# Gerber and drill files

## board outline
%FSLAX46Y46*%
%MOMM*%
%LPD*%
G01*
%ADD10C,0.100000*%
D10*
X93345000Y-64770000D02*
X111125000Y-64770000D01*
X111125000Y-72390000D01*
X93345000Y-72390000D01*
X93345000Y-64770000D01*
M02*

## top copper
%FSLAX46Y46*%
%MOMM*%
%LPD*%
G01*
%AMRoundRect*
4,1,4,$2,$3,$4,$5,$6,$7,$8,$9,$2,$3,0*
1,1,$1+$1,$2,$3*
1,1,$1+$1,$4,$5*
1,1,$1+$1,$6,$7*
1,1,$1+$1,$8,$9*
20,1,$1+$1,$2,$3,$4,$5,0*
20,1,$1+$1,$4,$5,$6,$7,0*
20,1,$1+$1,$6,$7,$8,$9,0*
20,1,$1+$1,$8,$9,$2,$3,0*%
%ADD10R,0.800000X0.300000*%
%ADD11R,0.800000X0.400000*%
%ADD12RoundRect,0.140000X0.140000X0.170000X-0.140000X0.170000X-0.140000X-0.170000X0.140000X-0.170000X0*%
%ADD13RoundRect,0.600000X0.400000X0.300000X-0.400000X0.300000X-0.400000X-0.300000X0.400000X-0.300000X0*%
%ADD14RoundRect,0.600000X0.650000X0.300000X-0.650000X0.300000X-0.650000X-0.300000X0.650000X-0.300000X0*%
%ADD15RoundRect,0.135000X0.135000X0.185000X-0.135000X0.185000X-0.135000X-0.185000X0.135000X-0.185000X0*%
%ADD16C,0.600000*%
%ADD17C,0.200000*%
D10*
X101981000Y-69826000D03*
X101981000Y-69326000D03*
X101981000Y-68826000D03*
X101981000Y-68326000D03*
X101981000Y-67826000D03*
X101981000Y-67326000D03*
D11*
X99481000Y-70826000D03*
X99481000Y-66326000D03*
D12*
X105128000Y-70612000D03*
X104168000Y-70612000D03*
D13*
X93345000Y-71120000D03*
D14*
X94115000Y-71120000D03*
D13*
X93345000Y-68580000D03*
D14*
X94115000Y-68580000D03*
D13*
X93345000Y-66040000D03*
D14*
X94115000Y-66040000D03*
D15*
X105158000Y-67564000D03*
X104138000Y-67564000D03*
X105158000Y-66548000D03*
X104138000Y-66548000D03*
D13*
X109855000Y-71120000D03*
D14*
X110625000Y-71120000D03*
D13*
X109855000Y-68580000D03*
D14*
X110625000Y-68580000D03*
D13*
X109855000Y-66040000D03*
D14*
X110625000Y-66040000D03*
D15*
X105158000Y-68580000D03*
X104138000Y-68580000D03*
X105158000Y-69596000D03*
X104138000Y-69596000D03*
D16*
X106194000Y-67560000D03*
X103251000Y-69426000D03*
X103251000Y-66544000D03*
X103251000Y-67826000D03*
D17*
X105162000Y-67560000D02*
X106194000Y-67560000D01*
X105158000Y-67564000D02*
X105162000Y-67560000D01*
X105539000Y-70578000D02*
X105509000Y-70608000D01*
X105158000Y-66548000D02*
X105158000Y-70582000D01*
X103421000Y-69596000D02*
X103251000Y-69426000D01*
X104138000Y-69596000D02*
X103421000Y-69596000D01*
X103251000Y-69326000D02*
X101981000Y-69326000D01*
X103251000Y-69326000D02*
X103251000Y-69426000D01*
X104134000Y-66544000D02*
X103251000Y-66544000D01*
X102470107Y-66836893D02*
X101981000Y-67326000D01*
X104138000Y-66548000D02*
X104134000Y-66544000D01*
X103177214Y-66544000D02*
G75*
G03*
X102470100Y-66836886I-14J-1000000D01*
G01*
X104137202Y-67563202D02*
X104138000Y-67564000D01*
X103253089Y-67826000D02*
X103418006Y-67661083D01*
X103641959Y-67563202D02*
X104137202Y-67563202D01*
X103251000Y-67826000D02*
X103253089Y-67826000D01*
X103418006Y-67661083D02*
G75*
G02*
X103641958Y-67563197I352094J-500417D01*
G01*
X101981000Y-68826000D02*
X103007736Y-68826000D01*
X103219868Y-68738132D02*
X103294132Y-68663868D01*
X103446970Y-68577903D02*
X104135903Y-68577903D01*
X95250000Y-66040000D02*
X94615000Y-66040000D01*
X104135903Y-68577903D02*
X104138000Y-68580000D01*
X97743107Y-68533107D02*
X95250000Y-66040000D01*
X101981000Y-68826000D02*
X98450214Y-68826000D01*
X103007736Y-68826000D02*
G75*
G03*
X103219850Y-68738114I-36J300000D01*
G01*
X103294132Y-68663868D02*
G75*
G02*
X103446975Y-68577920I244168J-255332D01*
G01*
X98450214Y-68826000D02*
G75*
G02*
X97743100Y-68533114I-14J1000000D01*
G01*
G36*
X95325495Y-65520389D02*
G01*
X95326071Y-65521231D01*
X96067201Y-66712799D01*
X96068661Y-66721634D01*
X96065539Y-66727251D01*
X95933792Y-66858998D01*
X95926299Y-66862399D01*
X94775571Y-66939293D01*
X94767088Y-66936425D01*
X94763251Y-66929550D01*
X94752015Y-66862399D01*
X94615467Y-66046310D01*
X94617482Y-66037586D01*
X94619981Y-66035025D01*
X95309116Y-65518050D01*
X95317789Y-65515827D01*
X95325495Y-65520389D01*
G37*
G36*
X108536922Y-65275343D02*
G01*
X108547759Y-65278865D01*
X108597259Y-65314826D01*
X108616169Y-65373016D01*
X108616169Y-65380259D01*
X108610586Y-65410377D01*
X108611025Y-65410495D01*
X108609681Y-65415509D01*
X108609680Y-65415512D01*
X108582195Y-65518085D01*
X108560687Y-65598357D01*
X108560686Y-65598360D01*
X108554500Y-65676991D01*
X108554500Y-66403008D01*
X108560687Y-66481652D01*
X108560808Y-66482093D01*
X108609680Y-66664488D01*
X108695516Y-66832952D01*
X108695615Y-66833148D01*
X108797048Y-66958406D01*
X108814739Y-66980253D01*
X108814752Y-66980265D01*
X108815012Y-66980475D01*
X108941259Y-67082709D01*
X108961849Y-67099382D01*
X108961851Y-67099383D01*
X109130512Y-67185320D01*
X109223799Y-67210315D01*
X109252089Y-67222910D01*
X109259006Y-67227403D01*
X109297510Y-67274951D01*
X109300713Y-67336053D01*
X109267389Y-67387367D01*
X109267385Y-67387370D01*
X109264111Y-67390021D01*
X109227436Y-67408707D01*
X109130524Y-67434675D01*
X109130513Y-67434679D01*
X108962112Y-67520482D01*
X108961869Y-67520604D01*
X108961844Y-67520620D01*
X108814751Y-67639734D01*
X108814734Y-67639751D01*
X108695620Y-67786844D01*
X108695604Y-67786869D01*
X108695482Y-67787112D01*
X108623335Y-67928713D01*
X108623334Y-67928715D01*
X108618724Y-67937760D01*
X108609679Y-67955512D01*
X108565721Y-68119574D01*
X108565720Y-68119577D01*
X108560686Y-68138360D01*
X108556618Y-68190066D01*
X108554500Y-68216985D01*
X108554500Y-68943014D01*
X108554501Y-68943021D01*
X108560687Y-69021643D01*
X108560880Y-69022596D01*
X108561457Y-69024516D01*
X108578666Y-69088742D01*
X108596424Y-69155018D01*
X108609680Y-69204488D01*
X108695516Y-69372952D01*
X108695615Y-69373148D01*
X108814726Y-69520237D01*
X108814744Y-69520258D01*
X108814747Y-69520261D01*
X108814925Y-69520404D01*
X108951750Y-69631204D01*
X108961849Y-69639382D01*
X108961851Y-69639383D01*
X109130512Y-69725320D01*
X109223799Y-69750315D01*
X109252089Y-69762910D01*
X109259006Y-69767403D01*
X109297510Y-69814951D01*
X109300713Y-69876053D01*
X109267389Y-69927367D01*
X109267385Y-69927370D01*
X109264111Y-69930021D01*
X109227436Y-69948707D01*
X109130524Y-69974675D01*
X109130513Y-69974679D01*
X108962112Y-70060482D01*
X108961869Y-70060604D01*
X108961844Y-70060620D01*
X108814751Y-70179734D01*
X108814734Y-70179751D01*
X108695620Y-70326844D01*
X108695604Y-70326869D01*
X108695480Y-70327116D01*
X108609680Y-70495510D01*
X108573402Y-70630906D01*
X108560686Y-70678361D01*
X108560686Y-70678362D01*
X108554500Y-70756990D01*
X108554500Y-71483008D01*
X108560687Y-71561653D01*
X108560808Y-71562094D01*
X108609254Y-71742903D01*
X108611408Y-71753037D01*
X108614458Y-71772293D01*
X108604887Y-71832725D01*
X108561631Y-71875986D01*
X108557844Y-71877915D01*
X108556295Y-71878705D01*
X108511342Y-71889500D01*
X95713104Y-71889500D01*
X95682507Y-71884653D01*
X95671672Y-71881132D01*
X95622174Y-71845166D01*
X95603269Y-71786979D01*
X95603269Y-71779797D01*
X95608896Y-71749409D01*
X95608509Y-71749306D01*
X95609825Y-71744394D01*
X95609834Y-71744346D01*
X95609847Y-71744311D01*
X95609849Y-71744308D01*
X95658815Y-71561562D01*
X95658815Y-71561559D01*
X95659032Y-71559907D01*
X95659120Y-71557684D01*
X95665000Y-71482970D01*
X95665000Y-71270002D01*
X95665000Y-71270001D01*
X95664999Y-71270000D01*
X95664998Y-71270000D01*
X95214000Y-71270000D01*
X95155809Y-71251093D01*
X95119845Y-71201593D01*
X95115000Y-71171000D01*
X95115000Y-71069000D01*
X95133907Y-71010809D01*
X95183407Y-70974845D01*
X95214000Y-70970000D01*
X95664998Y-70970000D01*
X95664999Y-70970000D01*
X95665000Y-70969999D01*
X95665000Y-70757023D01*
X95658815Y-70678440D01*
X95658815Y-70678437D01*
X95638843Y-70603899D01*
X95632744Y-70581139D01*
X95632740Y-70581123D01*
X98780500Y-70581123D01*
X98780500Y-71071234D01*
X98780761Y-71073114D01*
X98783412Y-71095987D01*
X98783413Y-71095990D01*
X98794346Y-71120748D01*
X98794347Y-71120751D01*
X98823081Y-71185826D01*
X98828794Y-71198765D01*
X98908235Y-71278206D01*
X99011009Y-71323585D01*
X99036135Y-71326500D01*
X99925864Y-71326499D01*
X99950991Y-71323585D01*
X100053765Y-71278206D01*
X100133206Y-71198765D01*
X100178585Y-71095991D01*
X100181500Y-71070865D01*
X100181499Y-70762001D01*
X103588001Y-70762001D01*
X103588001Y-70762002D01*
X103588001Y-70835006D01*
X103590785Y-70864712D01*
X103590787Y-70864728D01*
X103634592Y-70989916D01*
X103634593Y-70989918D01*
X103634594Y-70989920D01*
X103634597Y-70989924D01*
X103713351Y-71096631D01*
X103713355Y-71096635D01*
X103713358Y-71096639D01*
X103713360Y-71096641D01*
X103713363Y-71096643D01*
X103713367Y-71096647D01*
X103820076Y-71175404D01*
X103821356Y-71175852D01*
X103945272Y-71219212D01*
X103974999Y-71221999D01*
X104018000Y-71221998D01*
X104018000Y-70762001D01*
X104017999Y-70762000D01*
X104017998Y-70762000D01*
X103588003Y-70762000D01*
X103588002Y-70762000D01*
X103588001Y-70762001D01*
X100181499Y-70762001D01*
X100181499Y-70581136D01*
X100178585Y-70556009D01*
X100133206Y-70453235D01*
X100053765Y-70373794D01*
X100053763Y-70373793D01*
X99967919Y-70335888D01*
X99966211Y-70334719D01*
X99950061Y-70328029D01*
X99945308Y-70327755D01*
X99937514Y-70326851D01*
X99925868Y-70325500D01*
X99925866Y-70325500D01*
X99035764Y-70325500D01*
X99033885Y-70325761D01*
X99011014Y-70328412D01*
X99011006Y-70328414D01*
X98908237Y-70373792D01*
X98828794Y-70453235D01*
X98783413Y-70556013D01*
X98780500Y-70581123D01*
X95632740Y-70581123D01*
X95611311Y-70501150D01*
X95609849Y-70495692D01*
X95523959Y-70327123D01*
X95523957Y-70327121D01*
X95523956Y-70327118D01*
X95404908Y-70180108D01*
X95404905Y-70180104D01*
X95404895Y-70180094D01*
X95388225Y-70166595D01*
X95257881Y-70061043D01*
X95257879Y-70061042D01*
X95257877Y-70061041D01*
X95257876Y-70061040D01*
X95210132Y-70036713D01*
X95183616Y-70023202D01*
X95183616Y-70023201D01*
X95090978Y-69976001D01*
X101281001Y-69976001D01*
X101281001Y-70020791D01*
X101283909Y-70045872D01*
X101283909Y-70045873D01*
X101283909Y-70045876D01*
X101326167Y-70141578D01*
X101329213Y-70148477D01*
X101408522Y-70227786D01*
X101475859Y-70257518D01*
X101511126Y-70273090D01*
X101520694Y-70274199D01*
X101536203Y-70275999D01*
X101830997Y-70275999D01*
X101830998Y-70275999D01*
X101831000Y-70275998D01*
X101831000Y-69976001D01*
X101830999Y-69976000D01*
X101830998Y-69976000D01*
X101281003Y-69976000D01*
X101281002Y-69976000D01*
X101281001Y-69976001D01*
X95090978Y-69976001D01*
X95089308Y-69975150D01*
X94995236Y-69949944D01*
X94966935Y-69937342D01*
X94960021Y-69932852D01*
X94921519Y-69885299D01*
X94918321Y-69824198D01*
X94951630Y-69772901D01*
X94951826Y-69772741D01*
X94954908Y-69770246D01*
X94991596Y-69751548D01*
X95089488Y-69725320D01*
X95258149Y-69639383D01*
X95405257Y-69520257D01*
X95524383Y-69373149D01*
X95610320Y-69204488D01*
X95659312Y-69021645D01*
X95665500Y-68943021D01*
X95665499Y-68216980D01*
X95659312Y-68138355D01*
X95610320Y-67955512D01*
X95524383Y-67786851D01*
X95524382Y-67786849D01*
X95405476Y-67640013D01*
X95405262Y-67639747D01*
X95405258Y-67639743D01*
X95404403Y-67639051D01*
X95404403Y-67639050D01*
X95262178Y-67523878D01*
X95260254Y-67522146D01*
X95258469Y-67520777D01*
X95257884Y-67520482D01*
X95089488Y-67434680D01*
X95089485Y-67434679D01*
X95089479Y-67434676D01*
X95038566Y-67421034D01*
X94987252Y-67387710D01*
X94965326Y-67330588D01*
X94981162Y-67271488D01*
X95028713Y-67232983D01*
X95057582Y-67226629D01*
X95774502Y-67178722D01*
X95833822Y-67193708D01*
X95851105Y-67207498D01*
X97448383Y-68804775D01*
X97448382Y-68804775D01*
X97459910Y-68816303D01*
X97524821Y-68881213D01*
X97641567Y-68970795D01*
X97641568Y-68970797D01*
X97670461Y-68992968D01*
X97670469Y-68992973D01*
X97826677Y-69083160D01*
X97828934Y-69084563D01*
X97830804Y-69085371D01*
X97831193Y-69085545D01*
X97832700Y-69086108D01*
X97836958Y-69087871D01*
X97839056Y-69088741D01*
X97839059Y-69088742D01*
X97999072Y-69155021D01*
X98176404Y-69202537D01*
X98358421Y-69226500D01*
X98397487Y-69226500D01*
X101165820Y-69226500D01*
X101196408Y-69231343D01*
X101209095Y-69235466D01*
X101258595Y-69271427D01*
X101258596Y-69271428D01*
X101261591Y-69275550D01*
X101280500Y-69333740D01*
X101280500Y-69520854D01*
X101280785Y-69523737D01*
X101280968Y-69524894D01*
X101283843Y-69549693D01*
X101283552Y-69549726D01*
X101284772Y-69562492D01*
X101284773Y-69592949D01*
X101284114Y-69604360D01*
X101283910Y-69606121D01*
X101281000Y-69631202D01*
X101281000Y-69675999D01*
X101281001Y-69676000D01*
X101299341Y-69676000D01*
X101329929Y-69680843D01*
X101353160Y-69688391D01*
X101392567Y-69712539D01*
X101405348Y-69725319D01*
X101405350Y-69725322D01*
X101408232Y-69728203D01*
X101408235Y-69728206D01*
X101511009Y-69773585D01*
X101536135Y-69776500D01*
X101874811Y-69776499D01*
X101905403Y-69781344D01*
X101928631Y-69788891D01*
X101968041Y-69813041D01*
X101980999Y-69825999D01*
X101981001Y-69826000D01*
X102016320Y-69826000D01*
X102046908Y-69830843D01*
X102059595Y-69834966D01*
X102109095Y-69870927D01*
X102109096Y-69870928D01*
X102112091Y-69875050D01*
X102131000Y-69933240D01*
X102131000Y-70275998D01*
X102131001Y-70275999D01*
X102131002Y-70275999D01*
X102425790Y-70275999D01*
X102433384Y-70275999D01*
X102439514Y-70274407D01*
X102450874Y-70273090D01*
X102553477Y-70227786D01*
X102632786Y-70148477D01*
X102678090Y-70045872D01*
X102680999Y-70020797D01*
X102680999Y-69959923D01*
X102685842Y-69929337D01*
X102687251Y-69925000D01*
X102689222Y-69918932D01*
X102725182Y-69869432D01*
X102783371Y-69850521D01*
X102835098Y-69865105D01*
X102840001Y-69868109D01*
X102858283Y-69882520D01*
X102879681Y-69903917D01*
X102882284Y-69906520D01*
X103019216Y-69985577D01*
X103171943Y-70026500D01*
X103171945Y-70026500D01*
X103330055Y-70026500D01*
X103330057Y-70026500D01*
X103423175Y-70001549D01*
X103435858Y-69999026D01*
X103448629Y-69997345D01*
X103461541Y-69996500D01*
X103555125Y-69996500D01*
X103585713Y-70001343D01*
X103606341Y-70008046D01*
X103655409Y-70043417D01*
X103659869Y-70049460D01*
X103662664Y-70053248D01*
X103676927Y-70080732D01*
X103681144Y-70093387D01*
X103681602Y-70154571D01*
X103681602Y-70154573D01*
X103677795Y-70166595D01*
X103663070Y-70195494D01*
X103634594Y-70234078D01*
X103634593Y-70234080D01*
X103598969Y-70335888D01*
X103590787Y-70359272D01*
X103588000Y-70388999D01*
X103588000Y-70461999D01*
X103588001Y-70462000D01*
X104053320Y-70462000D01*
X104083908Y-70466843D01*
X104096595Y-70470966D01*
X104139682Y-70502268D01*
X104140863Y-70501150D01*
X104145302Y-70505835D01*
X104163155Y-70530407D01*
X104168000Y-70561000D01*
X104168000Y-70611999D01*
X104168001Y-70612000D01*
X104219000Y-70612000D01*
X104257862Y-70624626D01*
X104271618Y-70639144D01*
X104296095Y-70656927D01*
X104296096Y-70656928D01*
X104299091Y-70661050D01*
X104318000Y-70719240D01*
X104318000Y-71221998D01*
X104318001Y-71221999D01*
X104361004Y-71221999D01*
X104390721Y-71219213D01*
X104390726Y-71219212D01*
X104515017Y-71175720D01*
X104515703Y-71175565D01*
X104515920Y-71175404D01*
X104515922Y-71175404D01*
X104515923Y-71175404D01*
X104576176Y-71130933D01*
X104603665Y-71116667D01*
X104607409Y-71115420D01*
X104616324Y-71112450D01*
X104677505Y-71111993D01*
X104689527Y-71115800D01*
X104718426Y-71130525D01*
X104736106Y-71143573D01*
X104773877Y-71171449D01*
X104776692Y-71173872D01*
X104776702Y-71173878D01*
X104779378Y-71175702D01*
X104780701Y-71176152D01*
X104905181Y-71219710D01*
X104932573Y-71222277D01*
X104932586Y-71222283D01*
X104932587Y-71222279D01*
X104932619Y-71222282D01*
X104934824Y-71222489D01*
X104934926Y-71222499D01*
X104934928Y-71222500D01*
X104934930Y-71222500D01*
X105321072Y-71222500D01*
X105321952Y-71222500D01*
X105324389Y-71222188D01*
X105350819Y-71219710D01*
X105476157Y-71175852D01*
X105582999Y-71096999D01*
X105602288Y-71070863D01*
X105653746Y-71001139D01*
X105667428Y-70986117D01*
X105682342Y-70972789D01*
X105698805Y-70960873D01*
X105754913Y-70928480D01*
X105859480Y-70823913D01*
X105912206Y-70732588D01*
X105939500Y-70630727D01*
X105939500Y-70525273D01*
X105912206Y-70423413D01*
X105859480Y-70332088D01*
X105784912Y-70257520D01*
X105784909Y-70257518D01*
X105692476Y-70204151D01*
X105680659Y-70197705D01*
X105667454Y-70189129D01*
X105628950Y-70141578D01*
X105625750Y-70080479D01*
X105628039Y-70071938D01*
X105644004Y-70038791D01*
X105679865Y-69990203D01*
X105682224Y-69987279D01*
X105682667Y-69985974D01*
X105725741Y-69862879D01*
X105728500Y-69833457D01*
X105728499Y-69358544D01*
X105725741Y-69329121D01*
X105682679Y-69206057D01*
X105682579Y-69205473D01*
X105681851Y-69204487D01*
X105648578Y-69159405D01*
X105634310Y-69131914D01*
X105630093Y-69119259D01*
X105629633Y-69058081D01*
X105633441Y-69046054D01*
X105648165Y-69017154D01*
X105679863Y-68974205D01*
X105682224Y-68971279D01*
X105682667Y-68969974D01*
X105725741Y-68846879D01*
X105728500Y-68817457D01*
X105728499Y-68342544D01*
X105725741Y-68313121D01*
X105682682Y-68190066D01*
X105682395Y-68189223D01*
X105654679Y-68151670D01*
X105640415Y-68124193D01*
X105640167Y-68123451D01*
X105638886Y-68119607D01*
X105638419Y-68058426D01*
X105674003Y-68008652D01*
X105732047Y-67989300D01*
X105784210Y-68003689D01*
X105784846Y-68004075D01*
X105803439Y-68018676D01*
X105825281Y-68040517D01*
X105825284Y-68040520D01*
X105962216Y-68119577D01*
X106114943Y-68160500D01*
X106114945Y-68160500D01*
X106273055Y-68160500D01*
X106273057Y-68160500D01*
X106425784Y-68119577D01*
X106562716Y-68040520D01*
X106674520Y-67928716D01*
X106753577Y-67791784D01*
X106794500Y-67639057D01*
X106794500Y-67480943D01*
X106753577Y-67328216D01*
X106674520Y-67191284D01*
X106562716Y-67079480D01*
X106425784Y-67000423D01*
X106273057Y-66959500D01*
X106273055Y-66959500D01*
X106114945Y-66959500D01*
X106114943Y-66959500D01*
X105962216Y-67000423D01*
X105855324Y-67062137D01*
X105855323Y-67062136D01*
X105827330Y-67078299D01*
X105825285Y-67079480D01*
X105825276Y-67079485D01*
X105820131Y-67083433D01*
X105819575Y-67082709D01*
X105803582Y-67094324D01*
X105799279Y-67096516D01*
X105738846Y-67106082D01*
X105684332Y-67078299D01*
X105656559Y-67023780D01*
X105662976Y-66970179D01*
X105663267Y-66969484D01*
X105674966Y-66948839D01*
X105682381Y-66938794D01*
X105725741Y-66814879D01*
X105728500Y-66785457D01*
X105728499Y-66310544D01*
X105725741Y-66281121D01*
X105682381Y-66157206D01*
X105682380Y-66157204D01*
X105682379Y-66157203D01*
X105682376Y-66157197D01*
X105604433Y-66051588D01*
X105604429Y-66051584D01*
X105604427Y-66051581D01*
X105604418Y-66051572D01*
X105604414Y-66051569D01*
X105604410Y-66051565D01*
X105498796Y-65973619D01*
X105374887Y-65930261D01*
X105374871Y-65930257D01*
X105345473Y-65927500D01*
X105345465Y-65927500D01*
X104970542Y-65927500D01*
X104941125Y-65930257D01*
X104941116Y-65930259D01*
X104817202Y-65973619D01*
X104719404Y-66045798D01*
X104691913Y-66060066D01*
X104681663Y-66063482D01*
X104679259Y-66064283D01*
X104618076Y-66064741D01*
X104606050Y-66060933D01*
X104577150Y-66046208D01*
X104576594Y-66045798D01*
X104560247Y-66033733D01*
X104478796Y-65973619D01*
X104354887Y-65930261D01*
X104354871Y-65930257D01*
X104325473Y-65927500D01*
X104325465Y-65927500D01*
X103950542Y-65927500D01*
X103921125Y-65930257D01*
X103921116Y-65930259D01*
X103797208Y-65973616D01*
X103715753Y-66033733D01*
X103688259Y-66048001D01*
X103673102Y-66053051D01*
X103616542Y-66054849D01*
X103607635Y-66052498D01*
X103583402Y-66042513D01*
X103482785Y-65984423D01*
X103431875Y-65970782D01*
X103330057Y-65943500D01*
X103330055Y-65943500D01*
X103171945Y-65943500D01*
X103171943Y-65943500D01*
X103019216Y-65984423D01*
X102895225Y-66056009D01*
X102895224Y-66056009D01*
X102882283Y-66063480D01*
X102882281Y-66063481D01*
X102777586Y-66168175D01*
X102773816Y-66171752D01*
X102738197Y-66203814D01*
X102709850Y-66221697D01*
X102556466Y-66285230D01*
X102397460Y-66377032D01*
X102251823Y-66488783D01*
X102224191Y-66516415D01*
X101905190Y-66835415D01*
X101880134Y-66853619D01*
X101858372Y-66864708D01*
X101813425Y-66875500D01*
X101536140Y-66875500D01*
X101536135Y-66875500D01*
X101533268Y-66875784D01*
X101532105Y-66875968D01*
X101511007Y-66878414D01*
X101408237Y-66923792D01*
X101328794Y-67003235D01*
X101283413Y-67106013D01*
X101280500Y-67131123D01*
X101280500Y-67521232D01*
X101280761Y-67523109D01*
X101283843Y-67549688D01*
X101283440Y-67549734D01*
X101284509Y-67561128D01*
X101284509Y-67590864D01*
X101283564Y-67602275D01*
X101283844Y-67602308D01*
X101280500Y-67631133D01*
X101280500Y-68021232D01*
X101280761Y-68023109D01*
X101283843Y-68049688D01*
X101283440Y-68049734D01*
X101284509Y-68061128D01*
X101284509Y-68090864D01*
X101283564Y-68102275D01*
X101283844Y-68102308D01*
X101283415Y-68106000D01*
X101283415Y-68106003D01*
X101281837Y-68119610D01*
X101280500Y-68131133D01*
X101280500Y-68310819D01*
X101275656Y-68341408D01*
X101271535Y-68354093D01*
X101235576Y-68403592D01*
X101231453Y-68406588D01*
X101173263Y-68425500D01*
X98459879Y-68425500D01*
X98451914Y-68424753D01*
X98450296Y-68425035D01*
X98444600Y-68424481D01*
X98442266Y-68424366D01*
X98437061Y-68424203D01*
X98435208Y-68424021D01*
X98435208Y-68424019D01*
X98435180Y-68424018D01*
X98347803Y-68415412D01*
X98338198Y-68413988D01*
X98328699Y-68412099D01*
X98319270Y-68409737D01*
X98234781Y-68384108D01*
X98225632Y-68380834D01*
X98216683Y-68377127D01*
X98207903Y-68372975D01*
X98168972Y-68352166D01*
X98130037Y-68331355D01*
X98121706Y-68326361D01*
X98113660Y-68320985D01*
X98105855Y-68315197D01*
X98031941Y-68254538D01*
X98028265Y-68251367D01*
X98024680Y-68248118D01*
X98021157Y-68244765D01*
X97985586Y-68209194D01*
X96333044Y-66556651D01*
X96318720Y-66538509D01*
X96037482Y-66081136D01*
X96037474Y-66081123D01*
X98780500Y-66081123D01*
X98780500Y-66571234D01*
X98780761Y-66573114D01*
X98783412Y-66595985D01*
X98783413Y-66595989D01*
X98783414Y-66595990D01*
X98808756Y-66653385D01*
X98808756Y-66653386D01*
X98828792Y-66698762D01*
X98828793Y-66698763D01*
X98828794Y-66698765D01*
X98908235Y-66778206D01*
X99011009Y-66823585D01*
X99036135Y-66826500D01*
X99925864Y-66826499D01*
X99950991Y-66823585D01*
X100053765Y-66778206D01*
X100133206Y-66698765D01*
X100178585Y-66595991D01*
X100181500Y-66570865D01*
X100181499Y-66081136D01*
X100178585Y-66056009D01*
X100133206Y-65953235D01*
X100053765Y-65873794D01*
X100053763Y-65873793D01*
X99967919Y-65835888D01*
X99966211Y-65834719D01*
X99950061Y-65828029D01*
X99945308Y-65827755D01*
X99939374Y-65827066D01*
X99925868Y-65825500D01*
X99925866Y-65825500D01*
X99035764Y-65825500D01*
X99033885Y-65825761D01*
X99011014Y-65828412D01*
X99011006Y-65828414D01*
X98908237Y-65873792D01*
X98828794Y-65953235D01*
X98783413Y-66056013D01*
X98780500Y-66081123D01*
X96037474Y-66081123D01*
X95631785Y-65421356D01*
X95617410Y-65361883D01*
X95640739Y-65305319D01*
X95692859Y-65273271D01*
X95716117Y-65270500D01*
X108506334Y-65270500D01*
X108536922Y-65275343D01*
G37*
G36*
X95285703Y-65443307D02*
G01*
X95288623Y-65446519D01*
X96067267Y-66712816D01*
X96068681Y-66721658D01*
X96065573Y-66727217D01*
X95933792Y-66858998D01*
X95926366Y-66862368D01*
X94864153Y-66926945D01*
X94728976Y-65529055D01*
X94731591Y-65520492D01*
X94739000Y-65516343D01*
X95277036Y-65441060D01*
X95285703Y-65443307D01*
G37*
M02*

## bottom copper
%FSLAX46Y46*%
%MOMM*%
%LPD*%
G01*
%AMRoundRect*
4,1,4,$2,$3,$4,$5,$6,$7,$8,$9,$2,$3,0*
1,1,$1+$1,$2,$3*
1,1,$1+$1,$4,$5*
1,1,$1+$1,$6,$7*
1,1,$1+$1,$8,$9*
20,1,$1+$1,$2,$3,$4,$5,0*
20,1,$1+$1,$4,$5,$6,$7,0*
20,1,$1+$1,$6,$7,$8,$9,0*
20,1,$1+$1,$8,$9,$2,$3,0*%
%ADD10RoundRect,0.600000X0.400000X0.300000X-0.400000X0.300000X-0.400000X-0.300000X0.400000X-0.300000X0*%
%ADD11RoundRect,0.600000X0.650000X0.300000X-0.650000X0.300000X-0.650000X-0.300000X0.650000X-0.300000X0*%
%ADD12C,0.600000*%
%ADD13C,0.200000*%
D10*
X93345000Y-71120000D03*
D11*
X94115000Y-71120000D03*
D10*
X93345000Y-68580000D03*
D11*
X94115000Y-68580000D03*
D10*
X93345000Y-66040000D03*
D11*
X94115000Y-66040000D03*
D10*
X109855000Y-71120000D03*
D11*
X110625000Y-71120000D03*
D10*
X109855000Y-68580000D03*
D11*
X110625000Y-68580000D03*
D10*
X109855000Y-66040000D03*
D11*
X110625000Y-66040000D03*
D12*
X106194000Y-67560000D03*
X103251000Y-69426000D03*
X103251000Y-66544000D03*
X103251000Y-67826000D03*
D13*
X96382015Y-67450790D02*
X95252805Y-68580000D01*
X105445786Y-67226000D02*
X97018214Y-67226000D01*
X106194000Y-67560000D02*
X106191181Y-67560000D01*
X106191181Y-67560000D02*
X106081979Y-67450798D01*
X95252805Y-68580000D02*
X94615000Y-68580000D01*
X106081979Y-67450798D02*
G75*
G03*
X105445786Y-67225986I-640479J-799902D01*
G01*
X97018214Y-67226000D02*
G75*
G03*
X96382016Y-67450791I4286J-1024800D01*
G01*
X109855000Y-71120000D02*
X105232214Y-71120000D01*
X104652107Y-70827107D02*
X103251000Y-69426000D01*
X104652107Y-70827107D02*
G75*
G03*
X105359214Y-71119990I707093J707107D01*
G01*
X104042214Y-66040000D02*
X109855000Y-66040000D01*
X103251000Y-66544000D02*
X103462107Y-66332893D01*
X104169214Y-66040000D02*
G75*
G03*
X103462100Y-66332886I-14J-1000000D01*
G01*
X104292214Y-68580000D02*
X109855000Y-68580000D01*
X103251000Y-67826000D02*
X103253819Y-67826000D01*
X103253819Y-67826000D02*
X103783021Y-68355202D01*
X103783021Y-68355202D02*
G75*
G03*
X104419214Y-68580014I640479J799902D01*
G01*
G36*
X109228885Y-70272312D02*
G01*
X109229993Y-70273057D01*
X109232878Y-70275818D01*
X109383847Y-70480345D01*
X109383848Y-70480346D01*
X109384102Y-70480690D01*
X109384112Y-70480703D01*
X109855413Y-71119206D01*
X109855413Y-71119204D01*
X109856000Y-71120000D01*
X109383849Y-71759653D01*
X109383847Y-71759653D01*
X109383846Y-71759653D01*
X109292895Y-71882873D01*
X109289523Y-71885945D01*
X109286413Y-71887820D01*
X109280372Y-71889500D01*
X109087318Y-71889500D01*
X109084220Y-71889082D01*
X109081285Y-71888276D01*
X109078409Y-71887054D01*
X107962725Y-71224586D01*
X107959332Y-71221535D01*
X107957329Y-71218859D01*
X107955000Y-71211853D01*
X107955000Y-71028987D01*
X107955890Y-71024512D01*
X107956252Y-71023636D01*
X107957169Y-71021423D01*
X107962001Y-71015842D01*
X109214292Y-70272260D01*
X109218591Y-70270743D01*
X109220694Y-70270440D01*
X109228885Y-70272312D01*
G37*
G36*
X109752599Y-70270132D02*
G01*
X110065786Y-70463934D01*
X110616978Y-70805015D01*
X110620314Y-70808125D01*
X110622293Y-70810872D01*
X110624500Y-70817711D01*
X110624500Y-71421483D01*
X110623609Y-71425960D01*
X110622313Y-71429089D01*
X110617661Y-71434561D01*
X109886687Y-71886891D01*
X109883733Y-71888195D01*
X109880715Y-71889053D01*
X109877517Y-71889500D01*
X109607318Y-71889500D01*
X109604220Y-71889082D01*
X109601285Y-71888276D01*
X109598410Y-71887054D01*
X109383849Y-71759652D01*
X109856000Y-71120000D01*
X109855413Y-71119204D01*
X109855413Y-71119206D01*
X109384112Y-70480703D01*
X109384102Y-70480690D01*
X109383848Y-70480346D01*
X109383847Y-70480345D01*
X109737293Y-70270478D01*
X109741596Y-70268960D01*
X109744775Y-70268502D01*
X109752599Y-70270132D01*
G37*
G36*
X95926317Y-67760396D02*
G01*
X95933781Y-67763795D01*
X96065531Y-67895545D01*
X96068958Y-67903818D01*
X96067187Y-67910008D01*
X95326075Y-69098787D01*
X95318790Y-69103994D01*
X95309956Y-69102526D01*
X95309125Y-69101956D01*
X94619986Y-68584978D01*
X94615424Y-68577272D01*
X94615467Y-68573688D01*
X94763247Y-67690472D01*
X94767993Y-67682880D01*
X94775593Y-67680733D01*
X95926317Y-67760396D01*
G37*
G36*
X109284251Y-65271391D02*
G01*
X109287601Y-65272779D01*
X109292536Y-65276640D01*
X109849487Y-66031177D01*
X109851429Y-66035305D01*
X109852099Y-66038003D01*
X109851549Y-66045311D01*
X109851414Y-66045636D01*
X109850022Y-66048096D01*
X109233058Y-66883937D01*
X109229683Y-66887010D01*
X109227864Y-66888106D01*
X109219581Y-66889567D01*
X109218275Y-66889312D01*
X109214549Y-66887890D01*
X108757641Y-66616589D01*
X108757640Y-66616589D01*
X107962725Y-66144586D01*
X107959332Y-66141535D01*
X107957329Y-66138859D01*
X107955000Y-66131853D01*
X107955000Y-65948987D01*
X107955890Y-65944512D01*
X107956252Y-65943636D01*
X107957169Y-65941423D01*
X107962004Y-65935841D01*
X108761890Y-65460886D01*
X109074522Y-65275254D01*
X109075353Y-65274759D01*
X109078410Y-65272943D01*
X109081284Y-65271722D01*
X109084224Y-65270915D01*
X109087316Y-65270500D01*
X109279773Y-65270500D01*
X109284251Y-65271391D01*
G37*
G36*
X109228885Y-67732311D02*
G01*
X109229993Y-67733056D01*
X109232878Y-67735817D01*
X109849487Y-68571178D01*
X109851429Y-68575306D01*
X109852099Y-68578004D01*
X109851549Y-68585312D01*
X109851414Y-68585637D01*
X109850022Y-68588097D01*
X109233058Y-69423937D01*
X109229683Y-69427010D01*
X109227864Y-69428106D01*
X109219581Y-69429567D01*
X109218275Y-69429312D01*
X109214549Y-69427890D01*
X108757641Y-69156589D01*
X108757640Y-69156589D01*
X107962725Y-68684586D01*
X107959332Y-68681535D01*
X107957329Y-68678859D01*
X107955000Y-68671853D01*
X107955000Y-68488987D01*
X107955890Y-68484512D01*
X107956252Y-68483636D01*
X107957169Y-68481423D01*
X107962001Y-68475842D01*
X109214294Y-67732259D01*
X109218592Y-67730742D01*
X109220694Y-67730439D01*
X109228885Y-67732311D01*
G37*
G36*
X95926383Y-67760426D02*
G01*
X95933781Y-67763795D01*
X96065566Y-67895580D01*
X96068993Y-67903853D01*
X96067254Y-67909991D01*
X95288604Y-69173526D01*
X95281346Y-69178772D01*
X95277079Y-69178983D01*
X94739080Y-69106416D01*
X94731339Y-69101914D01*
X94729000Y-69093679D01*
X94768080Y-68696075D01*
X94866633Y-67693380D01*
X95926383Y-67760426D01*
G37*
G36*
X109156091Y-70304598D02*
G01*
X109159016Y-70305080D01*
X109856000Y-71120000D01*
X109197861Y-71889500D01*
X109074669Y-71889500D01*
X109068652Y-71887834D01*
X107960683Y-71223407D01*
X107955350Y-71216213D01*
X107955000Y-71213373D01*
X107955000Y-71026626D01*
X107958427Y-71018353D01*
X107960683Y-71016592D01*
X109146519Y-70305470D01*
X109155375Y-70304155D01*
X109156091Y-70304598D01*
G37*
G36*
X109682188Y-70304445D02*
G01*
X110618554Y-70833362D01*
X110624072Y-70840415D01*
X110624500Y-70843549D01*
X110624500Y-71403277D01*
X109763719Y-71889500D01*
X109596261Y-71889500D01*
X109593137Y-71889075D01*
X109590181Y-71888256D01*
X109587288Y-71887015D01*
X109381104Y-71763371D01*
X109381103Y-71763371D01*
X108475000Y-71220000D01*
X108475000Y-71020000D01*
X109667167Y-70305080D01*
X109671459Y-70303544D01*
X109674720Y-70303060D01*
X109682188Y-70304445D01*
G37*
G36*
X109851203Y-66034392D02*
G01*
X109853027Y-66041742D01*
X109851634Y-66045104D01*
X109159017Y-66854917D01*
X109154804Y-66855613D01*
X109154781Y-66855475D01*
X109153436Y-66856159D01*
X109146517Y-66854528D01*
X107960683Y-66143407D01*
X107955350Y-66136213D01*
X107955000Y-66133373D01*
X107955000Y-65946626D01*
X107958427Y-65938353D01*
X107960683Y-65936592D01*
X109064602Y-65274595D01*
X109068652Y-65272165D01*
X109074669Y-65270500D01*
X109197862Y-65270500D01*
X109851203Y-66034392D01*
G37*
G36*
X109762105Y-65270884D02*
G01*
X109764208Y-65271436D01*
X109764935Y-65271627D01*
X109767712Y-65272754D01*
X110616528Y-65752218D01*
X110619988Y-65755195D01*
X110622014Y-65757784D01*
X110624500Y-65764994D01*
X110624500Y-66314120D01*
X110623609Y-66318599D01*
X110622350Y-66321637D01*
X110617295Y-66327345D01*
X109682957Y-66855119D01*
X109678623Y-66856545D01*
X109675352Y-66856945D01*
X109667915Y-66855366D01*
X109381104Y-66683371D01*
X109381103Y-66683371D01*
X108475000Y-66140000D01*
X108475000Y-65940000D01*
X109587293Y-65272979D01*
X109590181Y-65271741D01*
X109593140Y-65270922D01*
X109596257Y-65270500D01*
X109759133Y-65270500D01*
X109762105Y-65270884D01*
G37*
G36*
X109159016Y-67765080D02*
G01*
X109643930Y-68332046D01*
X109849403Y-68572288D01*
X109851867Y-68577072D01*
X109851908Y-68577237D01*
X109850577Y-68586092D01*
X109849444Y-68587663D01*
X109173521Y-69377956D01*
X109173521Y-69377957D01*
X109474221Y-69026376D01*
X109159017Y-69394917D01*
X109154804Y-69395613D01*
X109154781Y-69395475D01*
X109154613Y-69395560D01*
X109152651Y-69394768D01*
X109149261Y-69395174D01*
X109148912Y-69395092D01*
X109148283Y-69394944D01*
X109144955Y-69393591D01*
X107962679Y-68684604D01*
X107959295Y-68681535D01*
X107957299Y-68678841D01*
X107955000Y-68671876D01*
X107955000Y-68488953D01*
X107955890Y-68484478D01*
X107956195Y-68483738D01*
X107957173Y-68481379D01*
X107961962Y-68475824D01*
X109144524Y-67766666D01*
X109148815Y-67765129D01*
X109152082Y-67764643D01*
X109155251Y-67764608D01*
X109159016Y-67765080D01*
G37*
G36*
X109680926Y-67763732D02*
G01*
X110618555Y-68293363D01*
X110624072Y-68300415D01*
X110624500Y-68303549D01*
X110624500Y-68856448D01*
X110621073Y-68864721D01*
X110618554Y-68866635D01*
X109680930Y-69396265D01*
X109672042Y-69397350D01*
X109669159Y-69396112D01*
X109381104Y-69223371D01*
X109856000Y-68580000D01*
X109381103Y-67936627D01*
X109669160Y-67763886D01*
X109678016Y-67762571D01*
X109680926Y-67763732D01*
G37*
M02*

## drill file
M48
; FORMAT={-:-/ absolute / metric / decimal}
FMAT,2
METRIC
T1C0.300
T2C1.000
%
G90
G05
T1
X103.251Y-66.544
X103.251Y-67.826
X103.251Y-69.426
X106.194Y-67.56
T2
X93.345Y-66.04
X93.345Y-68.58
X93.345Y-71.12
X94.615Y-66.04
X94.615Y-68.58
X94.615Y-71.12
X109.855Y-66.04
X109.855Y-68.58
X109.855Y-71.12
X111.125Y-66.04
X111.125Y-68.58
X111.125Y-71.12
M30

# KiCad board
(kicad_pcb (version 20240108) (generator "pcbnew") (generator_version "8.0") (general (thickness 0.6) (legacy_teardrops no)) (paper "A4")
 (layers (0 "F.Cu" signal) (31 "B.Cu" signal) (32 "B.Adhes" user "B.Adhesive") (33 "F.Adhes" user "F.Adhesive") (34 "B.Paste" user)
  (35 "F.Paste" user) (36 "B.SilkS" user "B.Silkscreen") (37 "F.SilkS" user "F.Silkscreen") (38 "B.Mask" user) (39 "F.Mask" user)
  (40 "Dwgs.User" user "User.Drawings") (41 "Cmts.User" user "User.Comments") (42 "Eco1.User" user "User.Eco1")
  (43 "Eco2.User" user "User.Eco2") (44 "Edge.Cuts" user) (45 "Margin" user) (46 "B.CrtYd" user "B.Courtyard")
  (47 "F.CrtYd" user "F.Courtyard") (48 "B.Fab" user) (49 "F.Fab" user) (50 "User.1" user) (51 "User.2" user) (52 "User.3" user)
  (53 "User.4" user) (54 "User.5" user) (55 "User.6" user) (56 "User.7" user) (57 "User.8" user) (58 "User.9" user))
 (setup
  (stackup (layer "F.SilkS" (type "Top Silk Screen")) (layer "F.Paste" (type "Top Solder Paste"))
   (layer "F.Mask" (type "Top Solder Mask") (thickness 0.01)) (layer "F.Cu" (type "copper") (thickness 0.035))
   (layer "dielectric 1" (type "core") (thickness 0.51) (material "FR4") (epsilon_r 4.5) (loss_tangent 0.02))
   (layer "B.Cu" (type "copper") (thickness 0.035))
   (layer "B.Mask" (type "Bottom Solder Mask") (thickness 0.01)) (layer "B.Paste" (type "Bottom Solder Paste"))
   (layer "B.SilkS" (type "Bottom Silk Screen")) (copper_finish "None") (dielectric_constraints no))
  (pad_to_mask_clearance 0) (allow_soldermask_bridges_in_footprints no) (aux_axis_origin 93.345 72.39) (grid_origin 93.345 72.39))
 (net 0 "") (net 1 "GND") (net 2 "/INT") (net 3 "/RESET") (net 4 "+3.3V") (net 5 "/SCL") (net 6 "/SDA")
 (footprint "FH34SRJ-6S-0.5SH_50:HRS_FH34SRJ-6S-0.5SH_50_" (layer "F.Cu") (at 100.731 68.576 -90)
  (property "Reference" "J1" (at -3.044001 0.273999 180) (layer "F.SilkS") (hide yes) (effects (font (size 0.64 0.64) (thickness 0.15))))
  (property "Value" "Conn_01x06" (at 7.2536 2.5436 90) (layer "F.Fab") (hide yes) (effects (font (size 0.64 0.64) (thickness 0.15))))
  (pad "1" smd rect (at 1.25 -1.25 270) (size 0.3 0.8) (layers "F.Cu" "F.Mask") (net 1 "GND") (solder_mask_margin 0.102)
   (teardrops (best_length_ratio 1) (max_length 1) (best_width_ratio 1) (max_width 2) (curve_points 10) (filter_ratio 0.9) (enabled no)
    (allow_two_segments yes) (prefer_zone_connections yes)))
  (pad "2" smd rect (at 0.75 -1.25 270) (size 0.3 0.8) (layers "F.Cu" "F.Mask") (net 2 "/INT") (solder_mask_margin 0.102)
   (teardrops (best_length_ratio 1) (max_length 1) (best_width_ratio 1) (max_width 2) (curve_points 10) (filter_ratio 0.9) (enabled no)
    (allow_two_segments yes) (prefer_zone_connections yes)))
  (pad "3" smd rect (at 0.25 -1.25 270) (size 0.3 0.8) (layers "F.Cu" "F.Mask") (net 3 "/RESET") (solder_mask_margin 0.102)
   (teardrops (best_length_ratio 1) (max_length 1) (best_width_ratio 1) (max_width 2) (curve_points 10) (filter_ratio 0.9) (enabled no)
    (allow_two_segments yes) (prefer_zone_connections yes)))
  (pad "4" smd rect (at -0.25 -1.25 270) (size 0.3 0.8) (layers "F.Cu" "F.Mask") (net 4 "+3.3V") (solder_mask_margin 0.102)
   (teardrops (best_length_ratio 1) (max_length 1) (best_width_ratio 1) (max_width 2) (curve_points 10) (filter_ratio 0.9) (enabled no)
    (allow_two_segments yes) (prefer_zone_connections yes)))
  (pad "5" smd rect (at -0.75 -1.25 270) (size 0.3 0.8) (layers "F.Cu" "F.Mask") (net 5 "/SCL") (solder_mask_margin 0.102)
   (teardrops (best_length_ratio 1) (max_length 1) (best_width_ratio 1) (max_width 2) (curve_points 10) (filter_ratio 0.9) (enabled no)
    (allow_two_segments yes) (prefer_zone_connections yes)))
  (pad "6" smd rect (at -1.25 -1.25 270) (size 0.3 0.8) (layers "F.Cu" "F.Mask") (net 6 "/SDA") (solder_mask_margin 0.102)
   (teardrops (best_length_ratio 1) (max_length 1) (best_width_ratio 1) (max_width 2) (curve_points 10) (filter_ratio 0.9) (enabled no)
    (allow_two_segments yes) (prefer_zone_connections yes)))
  (pad "S1" smd rect (at 2.25 1.25 270) (size 0.4 0.8) (layers "F.Cu" "F.Paste" "F.Mask") (solder_mask_margin 0.102)
   (teardrops (best_length_ratio 1) (max_length 1) (best_width_ratio 1) (max_width 2) (curve_points 10) (filter_ratio 0.9) (enabled no)
    (allow_two_segments yes) (prefer_zone_connections yes)))
  (pad "S2" smd rect (at -2.25 1.25 270) (size 0.4 0.8) (layers "F.Cu" "F.Paste" "F.Mask") (solder_mask_margin 0.102)
   (teardrops (best_length_ratio 1) (max_length 1) (best_width_ratio 1) (max_width 2) (curve_points 10) (filter_ratio 0.9) (enabled no)
    (allow_two_segments yes) (prefer_zone_connections yes))))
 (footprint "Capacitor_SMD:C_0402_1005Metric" (layer "F.Cu") (at 104.648 70.612 180)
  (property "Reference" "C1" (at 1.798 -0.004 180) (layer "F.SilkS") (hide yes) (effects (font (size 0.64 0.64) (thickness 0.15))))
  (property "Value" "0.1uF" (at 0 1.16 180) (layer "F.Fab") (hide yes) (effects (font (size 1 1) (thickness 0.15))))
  (pad "1" smd roundrect (at -0.48 0 180) (size 0.56 0.62) (layers "F.Cu" "F.Paste" "F.Mask") (roundrect_rratio 0.25) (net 4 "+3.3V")
   (teardrops (best_length_ratio 1) (max_length 1) (best_width_ratio 1) (max_width 2) (curve_points 10) (filter_ratio 0.9) (enabled no)
    (allow_two_segments yes) (prefer_zone_connections yes)))
  (pad "2" smd roundrect (at 0.48 0 180) (size 0.56 0.62) (layers "F.Cu" "F.Paste" "F.Mask") (roundrect_rratio 0.25) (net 1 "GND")
   (teardrops (best_length_ratio 1) (max_length 1) (best_width_ratio 1) (max_width 2) (curve_points 10) (filter_ratio 0.9) (enabled no)
    (allow_two_segments yes) (prefer_zone_connections yes))))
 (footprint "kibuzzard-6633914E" (layer "F.Cu") (at 107.442 71.12)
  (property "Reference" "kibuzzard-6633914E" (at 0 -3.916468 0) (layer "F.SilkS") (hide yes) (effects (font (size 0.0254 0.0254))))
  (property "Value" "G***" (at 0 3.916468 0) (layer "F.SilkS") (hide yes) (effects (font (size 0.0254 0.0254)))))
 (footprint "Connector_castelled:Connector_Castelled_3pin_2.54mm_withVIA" (layer "F.Cu") (at 93.345 71.12 90)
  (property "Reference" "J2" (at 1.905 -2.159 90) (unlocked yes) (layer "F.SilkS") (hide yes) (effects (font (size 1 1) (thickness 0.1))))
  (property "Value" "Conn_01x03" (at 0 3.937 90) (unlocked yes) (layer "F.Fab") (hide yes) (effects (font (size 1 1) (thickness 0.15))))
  (pad "1" thru_hole roundrect (at 0 0 180) (size 2 1.8) (drill 1) (layers "*.Cu" "*.Mask") (remove_unused_layers no)
   (roundrect_rratio 0.3333333333) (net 1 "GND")
   (teardrops (best_length_ratio 0.5) (max_length 1) (best_width_ratio 1) (max_width 2) (curve_points 0) (filter_ratio 0.9) (enabled yes)
    (allow_two_segments yes) (prefer_zone_connections yes)))
  (pad "1" thru_hole roundrect (at 0 1.27 180) (size 2.5 1.8) (drill 1 (offset 0.5 0)) (layers "*.Cu" "*.Mask") (remove_unused_layers no)
   (roundrect_rratio 0.3333333333) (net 1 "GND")
   (teardrops (best_length_ratio 0.5) (max_length 1) (best_width_ratio 1) (max_width 2) (curve_points 0) (filter_ratio 0.9) (enabled yes)
    (allow_two_segments yes) (prefer_zone_connections yes)))
  (pad "2" thru_hole roundrect (at 2.54 0 180) (size 2 1.8) (drill 1) (layers "*.Cu" "*.Mask") (remove_unused_layers no)
   (roundrect_rratio 0.3333333333) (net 4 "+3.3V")
   (teardrops (best_length_ratio 0.5) (max_length 1) (best_width_ratio 1) (max_width 2) (curve_points 0) (filter_ratio 0.9) (enabled yes)
    (allow_two_segments yes) (prefer_zone_connections yes)))
  (pad "2" thru_hole roundrect (at 2.54 1.27 180) (size 2.5 1.8) (drill 1 (offset 0.5 0)) (layers "*.Cu" "*.Mask") (remove_unused_layers no)
   (roundrect_rratio 0.3333333333) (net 4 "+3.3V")
   (teardrops (best_length_ratio 0.5) (max_length 1) (best_width_ratio 1) (max_width 2) (curve_points 0) (filter_ratio 0.9) (enabled yes)
    (allow_two_segments yes) (prefer_zone_connections yes)))
  (pad "3" thru_hole roundrect (at 5.08 0 180) (size 2 1.8) (drill 1) (layers "*.Cu" "*.Mask") (remove_unused_layers no)
   (roundrect_rratio 0.3333333333) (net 3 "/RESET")
   (teardrops (best_length_ratio 0.5) (max_length 1) (best_width_ratio 1) (max_width 2) (curve_points 0) (filter_ratio 0.9) (enabled yes)
    (allow_two_segments yes) (prefer_zone_connections yes)))
  (pad "3" thru_hole roundrect (at 5.08 1.27 180) (size 2.5 1.8) (drill 1 (offset 0.5 0)) (layers "*.Cu" "*.Mask") (remove_unused_layers no)
   (roundrect_rratio 0.3333333333) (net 3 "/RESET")
   (teardrops (best_length_ratio 0.5) (max_length 1) (best_width_ratio 1) (max_width 2) (curve_points 0) (filter_ratio 0.9) (enabled yes)
    (allow_two_segments yes) (prefer_zone_connections yes))))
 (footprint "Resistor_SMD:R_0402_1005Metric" (layer "F.Cu") (at 104.648 67.564 180)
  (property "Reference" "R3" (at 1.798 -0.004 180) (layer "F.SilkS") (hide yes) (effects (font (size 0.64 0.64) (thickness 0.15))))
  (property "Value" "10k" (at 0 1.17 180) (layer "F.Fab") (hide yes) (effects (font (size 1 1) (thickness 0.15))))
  (pad "1" smd roundrect (at -0.51 0 180) (size 0.54 0.64) (layers "F.Cu" "F.Paste" "F.Mask") (roundrect_rratio 0.25) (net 4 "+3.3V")
   (teardrops (best_length_ratio 1) (max_length 1) (best_width_ratio 1) (max_width 2) (curve_points 10) (filter_ratio 0.9) (enabled no)
    (allow_two_segments yes) (prefer_zone_connections yes)))
  (pad "2" smd roundrect (at 0.51 0 180) (size 0.54 0.64) (layers "F.Cu" "F.Paste" "F.Mask") (roundrect_rratio 0.25) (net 5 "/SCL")
   (teardrops (best_length_ratio 1) (max_length 1) (best_width_ratio 1) (max_width 2) (curve_points 10) (filter_ratio 0.9) (enabled no)
    (allow_two_segments yes) (prefer_zone_connections yes))))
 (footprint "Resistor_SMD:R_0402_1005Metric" (layer "F.Cu") (at 104.648 66.548 180)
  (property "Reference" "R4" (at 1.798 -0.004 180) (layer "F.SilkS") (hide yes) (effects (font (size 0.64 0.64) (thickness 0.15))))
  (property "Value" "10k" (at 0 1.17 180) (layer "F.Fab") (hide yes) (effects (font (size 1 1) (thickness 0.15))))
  (pad "1" smd roundrect (at -0.51 0 180) (size 0.54 0.64) (layers "F.Cu" "F.Paste" "F.Mask") (roundrect_rratio 0.25) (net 4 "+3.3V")
   (teardrops (best_length_ratio 1) (max_length 1) (best_width_ratio 1) (max_width 2) (curve_points 10) (filter_ratio 0.9) (enabled no)
    (allow_two_segments yes) (prefer_zone_connections yes)))
  (pad "2" smd roundrect (at 0.51 0 180) (size 0.54 0.64) (layers "F.Cu" "F.Paste" "F.Mask") (roundrect_rratio 0.25) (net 6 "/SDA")
   (teardrops (best_length_ratio 1) (max_length 1) (best_width_ratio 1) (max_width 2) (curve_points 10) (filter_ratio 0.9) (enabled no)
    (allow_two_segments yes) (prefer_zone_connections yes))))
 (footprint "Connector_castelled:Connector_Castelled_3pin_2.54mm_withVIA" (layer "F.Cu") (at 109.855 71.12 90)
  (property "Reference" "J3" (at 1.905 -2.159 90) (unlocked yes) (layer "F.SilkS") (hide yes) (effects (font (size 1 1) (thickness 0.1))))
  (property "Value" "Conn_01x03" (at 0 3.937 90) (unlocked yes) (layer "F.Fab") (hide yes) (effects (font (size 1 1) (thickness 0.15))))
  (pad "1" thru_hole roundrect (at 0 0 180) (size 2 1.8) (drill 1) (layers "*.Cu" "*.Mask") (remove_unused_layers no)
   (roundrect_rratio 0.3333333333) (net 2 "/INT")
   (teardrops (best_length_ratio 0.5) (max_length 1) (best_width_ratio 1) (max_width 2) (curve_points 0) (filter_ratio 0.9) (enabled yes)
    (allow_two_segments yes) (prefer_zone_connections yes)))
  (pad "1" thru_hole roundrect (at 0 1.27 180) (size 2.5 1.8) (drill 1 (offset 0.5 0)) (layers "*.Cu" "*.Mask") (remove_unused_layers no)
   (roundrect_rratio 0.3333333333) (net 2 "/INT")
   (teardrops (best_length_ratio 0.5) (max_length 1) (best_width_ratio 1) (max_width 2) (curve_points 0) (filter_ratio 0.9) (enabled yes)
    (allow_two_segments yes) (prefer_zone_connections yes)))
  (pad "2" thru_hole roundrect (at 2.54 0 180) (size 2 1.8) (drill 1) (layers "*.Cu" "*.Mask") (remove_unused_layers no)
   (roundrect_rratio 0.3333333333) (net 5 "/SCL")
   (teardrops (best_length_ratio 0.5) (max_length 1) (best_width_ratio 1) (max_width 2) (curve_points 0) (filter_ratio 0.9) (enabled yes)
    (allow_two_segments yes) (prefer_zone_connections yes)))
  (pad "2" thru_hole roundrect (at 2.54 1.27 180) (size 2.5 1.8) (drill 1 (offset 0.5 0)) (layers "*.Cu" "*.Mask") (remove_unused_layers no)
   (roundrect_rratio 0.3333333333) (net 5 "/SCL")
   (teardrops (best_length_ratio 0.5) (max_length 1) (best_width_ratio 1) (max_width 2) (curve_points 0) (filter_ratio 0.9) (enabled yes)
    (allow_two_segments yes) (prefer_zone_connections yes)))
  (pad "3" thru_hole roundrect (at 5.08 0 180) (size 2 1.8) (drill 1) (layers "*.Cu" "*.Mask") (remove_unused_layers no)
   (roundrect_rratio 0.3333333333) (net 6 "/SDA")
   (teardrops (best_length_ratio 0.5) (max_length 1) (best_width_ratio 1) (max_width 2) (curve_points 0) (filter_ratio 0.9) (enabled yes)
    (allow_two_segments yes) (prefer_zone_connections yes)))
  (pad "3" thru_hole roundrect (at 5.08 1.27 180) (size 2.5 1.8) (drill 1 (offset 0.5 0)) (layers "*.Cu" "*.Mask") (remove_unused_layers no)
   (roundrect_rratio 0.3333333333) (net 6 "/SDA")
   (teardrops (best_length_ratio 0.5) (max_length 1) (best_width_ratio 1) (max_width 2) (curve_points 0) (filter_ratio 0.9) (enabled yes)
    (allow_two_segments yes) (prefer_zone_connections yes))))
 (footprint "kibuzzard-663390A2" (layer "F.Cu") (at 96.774 66.04)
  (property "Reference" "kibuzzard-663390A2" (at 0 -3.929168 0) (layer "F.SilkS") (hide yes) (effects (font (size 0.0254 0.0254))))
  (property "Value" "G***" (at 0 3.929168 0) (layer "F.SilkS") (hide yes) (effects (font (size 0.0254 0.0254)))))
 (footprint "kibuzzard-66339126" (layer "F.Cu") (at 107.442 68.58)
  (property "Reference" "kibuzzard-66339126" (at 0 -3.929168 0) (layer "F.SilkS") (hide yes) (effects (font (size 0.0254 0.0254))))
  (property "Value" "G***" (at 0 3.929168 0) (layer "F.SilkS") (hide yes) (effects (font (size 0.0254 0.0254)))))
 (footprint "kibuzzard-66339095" (layer "F.Cu") (at 96.901 71.12)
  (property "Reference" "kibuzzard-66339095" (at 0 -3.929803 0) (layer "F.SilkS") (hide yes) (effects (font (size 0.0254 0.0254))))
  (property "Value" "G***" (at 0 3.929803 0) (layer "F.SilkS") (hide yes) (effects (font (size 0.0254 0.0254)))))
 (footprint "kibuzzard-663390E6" (layer "F.Cu") (at 107.442 66.04)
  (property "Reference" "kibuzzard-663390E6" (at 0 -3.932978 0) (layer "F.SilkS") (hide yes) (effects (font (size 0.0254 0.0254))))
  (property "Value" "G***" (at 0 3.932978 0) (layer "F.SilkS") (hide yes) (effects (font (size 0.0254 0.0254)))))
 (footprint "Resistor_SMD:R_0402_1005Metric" (layer "F.Cu") (at 104.648 68.58 180)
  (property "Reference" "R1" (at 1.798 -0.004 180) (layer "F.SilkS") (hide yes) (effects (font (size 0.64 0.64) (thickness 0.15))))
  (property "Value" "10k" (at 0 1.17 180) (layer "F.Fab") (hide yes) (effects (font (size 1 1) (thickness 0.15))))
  (pad "1" smd roundrect (at -0.51 0 180) (size 0.54 0.64) (layers "F.Cu" "F.Paste" "F.Mask") (roundrect_rratio 0.25) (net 4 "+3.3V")
   (teardrops (best_length_ratio 1) (max_length 1) (best_width_ratio 1) (max_width 2) (curve_points 10) (filter_ratio 0.9) (enabled no)
    (allow_two_segments yes) (prefer_zone_connections yes)))
  (pad "2" smd roundrect (at 0.51 0 180) (size 0.54 0.64) (layers "F.Cu" "F.Paste" "F.Mask") (roundrect_rratio 0.25) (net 3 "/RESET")
   (teardrops (best_length_ratio 1) (max_length 1) (best_width_ratio 1) (max_width 2) (curve_points 10) (filter_ratio 0.9) (enabled no)
    (allow_two_segments yes) (prefer_zone_connections yes))))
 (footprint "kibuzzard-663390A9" (layer "F.Cu") (at 96.774 68.58)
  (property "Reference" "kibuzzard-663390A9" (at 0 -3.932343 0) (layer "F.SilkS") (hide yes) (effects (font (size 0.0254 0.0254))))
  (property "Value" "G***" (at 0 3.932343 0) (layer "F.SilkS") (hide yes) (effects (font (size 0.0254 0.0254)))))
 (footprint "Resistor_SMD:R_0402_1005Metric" (layer "F.Cu") (at 104.648 69.596 180)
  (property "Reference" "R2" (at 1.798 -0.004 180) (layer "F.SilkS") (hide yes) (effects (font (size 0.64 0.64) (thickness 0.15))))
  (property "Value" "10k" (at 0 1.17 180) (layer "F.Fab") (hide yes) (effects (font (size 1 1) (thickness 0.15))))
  (pad "1" smd roundrect (at -0.51 0 180) (size 0.54 0.64) (layers "F.Cu" "F.Paste" "F.Mask") (roundrect_rratio 0.25) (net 4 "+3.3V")
   (teardrops (best_length_ratio 1) (max_length 1) (best_width_ratio 1) (max_width 2) (curve_points 10) (filter_ratio 0.9) (enabled no)
    (allow_two_segments yes) (prefer_zone_connections yes)))
  (pad "2" smd roundrect (at 0.51 0 180) (size 0.54 0.64) (layers "F.Cu" "F.Paste" "F.Mask") (roundrect_rratio 0.25) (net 2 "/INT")
   (teardrops (best_length_ratio 1) (max_length 1) (best_width_ratio 1) (max_width 2) (curve_points 10) (filter_ratio 0.9) (enabled no)
    (allow_two_segments yes) (prefer_zone_connections yes))))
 (gr_rect (start 93.345 64.77) (end 111.125 72.39) (stroke (width 0.1) (type default)) (fill none) (layer "Edge.Cuts"))
 (segment (start 105.162 67.56) (end 106.194 67.56) (width 0.2) (layer "F.Cu") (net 4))
 (segment (start 105.158 67.564) (end 105.162 67.56) (width 0.2) (layer "F.Cu") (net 4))
 (segment (start 105.539 70.578) (end 105.509 70.608) (width 0.2) (layer "F.Cu") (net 4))
 (segment (start 105.158 66.548) (end 105.158 70.582) (width 0.2) (layer "F.Cu") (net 4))
 (via (at 106.194 67.56) (size 0.6) (drill 0.3) (layers "F.Cu" "B.Cu")
  (teardrops (best_length_ratio 1) (max_length 1) (best_width_ratio 1) (max_width 2) (curve_points 10) (filter_ratio 0.9) (enabled no)
   (allow_two_segments yes) (prefer_zone_connections yes))
  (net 4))
 (segment (start 96.382015 67.45079) (end 95.252805 68.58) (width 0.2) (layer "B.Cu") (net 4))
 (segment (start 105.445786 67.226) (end 97.018214 67.226) (width 0.2) (layer "B.Cu") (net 4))
 (segment (start 106.194 67.56) (end 106.191181 67.56) (width 0.2) (layer "B.Cu") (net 4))
 (segment (start 106.191181 67.56) (end 106.081979 67.450798) (width 0.2) (layer "B.Cu") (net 4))
 (segment (start 95.252805 68.58) (end 94.615 68.58) (width 0.2) (layer "B.Cu") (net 4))
 (arc (start 106.081979 67.450798) (mid 105.782679 67.284452) (end 105.445786 67.226) (width 0.2) (layer "B.Cu") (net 4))
 (arc (start 97.018214 67.226) (mid 96.681322 67.284452) (end 96.382015 67.45079) (width 0.2) (layer "B.Cu") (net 4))
 (segment (start 103.421 69.596) (end 103.251 69.426) (width 0.2) (layer "F.Cu") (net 2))
 (segment (start 104.138 69.596) (end 103.421 69.596) (width 0.2) (layer "F.Cu") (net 2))
 (segment (start 103.251 69.326) (end 101.981 69.326) (width 0.2) (layer "F.Cu") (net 2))
 (segment (start 103.251 69.326) (end 103.251 69.426) (width 0.2) (layer "F.Cu") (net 2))
 (via (at 103.251 69.426) (size 0.6) (drill 0.3) (layers "F.Cu" "B.Cu")
  (teardrops (best_length_ratio 1) (max_length 1) (best_width_ratio 1) (max_width 2) (curve_points 10) (filter_ratio 0.9) (enabled no)
   (allow_two_segments yes) (prefer_zone_connections yes))
  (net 2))
 (segment (start 109.855 71.12) (end 105.232214 71.12) (width 0.2) (layer "B.Cu") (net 2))
 (segment (start 104.652107 70.827107) (end 103.251 69.426) (width 0.2) (layer "B.Cu") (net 2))
 (arc (start 104.652107 70.827107) (mid 104.97653 71.04388) (end 105.359214 71.12) (width 0.2) (layer "B.Cu") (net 2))
 (segment (start 104.134 66.544) (end 103.251 66.544) (width 0.2) (layer "F.Cu") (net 6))
 (segment (start 102.470107 66.836893) (end 101.981 67.326) (width 0.2) (layer "F.Cu") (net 6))
 (segment (start 104.138 66.548) (end 104.134 66.544) (width 0.2) (layer "F.Cu") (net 6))
 (via (at 103.251 66.544) (size 0.6) (drill 0.3) (layers "F.Cu" "B.Cu")
  (teardrops (best_length_ratio 1) (max_length 1) (best_width_ratio 1) (max_width 2) (curve_points 10) (filter_ratio 0.9) (enabled no)
   (allow_two_segments yes) (prefer_zone_connections yes))
  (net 6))
 (arc (start 103.177214 66.544) (mid 102.794531 66.62012) (end 102.470107 66.836893) (width 0.2) (layer "F.Cu") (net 6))
 (segment (start 104.042214 66.04) (end 109.855 66.04) (width 0.2) (layer "B.Cu") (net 6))
 (segment (start 103.251 66.544) (end 103.462107 66.332893) (width 0.2) (layer "B.Cu") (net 6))
 (arc (start 104.169214 66.04) (mid 103.786531 66.11612) (end 103.462107 66.332893) (width 0.2) (layer "B.Cu") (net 6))
 (segment (start 104.137202 67.563202) (end 104.138 67.564) (width 0.2) (layer "F.Cu") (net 5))
 (segment (start 103.253089 67.826) (end 103.418006 67.661083) (width 0.2) (layer "F.Cu") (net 5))
 (segment (start 103.641959 67.563202) (end 104.137202 67.563202) (width 0.2) (layer "F.Cu") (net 5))
 (segment (start 103.251 67.826) (end 103.253089 67.826) (width 0.2) (layer "F.Cu") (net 5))
 (via (at 103.251 67.826) (size 0.6) (drill 0.3) (layers "F.Cu" "B.Cu")
  (teardrops (best_length_ratio 1) (max_length 1) (best_width_ratio 1) (max_width 2) (curve_points 10) (filter_ratio 0.9) (enabled no)
   (allow_two_segments yes) (prefer_zone_connections yes))
  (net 5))
 (arc (start 103.418006 67.661083) (mid 103.524808 67.600951) (end 103.641959 67.563202) (width 0.2) (layer "F.Cu") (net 5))
 (segment (start 104.292214 68.58) (end 109.855 68.58) (width 0.2) (layer "B.Cu") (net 5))
 (segment (start 103.251 67.826) (end 103.253819 67.826) (width 0.2) (layer "B.Cu") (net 5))
 (segment (start 103.253819 67.826) (end 103.783021 68.355202) (width 0.2) (layer "B.Cu") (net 5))
 (arc (start 103.783021 68.355202) (mid 104.082321 68.521548) (end 104.419214 68.58) (width 0.2) (layer "B.Cu") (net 5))
 (segment (start 101.981 68.826) (end 103.007736 68.826) (width 0.2) (layer "F.Cu") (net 3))
 (segment (start 103.219868 68.738132) (end 103.294132 68.663868) (width 0.2) (layer "F.Cu") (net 3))
 (segment (start 103.44697 68.577903) (end 104.135903 68.577903) (width 0.2) (layer "F.Cu") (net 3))
 (segment (start 95.25 66.04) (end 94.615 66.04) (width 0.2) (layer "F.Cu") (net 3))
 (segment (start 104.135903 68.577903) (end 104.138 68.58) (width 0.2) (layer "F.Cu") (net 3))
 (segment (start 97.743107 68.533107) (end 95.25 66.04) (width 0.2) (layer "F.Cu") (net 3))
 (segment (start 101.981 68.826) (end 98.450214 68.826) (width 0.2) (layer "F.Cu") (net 3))
 (arc (start 103.007736 68.826) (mid 103.122541 68.803164) (end 103.219868 68.738132) (width 0.2) (layer "F.Cu") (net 3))
 (arc (start 103.294132 68.663868) (mid 103.364843 68.611415) (end 103.44697 68.577903) (width 0.2) (layer "F.Cu") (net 3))
 (arc (start 98.450214 68.826) (mid 98.067531 68.74988) (end 97.743107 68.533107) (width 0.2) (layer "F.Cu") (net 3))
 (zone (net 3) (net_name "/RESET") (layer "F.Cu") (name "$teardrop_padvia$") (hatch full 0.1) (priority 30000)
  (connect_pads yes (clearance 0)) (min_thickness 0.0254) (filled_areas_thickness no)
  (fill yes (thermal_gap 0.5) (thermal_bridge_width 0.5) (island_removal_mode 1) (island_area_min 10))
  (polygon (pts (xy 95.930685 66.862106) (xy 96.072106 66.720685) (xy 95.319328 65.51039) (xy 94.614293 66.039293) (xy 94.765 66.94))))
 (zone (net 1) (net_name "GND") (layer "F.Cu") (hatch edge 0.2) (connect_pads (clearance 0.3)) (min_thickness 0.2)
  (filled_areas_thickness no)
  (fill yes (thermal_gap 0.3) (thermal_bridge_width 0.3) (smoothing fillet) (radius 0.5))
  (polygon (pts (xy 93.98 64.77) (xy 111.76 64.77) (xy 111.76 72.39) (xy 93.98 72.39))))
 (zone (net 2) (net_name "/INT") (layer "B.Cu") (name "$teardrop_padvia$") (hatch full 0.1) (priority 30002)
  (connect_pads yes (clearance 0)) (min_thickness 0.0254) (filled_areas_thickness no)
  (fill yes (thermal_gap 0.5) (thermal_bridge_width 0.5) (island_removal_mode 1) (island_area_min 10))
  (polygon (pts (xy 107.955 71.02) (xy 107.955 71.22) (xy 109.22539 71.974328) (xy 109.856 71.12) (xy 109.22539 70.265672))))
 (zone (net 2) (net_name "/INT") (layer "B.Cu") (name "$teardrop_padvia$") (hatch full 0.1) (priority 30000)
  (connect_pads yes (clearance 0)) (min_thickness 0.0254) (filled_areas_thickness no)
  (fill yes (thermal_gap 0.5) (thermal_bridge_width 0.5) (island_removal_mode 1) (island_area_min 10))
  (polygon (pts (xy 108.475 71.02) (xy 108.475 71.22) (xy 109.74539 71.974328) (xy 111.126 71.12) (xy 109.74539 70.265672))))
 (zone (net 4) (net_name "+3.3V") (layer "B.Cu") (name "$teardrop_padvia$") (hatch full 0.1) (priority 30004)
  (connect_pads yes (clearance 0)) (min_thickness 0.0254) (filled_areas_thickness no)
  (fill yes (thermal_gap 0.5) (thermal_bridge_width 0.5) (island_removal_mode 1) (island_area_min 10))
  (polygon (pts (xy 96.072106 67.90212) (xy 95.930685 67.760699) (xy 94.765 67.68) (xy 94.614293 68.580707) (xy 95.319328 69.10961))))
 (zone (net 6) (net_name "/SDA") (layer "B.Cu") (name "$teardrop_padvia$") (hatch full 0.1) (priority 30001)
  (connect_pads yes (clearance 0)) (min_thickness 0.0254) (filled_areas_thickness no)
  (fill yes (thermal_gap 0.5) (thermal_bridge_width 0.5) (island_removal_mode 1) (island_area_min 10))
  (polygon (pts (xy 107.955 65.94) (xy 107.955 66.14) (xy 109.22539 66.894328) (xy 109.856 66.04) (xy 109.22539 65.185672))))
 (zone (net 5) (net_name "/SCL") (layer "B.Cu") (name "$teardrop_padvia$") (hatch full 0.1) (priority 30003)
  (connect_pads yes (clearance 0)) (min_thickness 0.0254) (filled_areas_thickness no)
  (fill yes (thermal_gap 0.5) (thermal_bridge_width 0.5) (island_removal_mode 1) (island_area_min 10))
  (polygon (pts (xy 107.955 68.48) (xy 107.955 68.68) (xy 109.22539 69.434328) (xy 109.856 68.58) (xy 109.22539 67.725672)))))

